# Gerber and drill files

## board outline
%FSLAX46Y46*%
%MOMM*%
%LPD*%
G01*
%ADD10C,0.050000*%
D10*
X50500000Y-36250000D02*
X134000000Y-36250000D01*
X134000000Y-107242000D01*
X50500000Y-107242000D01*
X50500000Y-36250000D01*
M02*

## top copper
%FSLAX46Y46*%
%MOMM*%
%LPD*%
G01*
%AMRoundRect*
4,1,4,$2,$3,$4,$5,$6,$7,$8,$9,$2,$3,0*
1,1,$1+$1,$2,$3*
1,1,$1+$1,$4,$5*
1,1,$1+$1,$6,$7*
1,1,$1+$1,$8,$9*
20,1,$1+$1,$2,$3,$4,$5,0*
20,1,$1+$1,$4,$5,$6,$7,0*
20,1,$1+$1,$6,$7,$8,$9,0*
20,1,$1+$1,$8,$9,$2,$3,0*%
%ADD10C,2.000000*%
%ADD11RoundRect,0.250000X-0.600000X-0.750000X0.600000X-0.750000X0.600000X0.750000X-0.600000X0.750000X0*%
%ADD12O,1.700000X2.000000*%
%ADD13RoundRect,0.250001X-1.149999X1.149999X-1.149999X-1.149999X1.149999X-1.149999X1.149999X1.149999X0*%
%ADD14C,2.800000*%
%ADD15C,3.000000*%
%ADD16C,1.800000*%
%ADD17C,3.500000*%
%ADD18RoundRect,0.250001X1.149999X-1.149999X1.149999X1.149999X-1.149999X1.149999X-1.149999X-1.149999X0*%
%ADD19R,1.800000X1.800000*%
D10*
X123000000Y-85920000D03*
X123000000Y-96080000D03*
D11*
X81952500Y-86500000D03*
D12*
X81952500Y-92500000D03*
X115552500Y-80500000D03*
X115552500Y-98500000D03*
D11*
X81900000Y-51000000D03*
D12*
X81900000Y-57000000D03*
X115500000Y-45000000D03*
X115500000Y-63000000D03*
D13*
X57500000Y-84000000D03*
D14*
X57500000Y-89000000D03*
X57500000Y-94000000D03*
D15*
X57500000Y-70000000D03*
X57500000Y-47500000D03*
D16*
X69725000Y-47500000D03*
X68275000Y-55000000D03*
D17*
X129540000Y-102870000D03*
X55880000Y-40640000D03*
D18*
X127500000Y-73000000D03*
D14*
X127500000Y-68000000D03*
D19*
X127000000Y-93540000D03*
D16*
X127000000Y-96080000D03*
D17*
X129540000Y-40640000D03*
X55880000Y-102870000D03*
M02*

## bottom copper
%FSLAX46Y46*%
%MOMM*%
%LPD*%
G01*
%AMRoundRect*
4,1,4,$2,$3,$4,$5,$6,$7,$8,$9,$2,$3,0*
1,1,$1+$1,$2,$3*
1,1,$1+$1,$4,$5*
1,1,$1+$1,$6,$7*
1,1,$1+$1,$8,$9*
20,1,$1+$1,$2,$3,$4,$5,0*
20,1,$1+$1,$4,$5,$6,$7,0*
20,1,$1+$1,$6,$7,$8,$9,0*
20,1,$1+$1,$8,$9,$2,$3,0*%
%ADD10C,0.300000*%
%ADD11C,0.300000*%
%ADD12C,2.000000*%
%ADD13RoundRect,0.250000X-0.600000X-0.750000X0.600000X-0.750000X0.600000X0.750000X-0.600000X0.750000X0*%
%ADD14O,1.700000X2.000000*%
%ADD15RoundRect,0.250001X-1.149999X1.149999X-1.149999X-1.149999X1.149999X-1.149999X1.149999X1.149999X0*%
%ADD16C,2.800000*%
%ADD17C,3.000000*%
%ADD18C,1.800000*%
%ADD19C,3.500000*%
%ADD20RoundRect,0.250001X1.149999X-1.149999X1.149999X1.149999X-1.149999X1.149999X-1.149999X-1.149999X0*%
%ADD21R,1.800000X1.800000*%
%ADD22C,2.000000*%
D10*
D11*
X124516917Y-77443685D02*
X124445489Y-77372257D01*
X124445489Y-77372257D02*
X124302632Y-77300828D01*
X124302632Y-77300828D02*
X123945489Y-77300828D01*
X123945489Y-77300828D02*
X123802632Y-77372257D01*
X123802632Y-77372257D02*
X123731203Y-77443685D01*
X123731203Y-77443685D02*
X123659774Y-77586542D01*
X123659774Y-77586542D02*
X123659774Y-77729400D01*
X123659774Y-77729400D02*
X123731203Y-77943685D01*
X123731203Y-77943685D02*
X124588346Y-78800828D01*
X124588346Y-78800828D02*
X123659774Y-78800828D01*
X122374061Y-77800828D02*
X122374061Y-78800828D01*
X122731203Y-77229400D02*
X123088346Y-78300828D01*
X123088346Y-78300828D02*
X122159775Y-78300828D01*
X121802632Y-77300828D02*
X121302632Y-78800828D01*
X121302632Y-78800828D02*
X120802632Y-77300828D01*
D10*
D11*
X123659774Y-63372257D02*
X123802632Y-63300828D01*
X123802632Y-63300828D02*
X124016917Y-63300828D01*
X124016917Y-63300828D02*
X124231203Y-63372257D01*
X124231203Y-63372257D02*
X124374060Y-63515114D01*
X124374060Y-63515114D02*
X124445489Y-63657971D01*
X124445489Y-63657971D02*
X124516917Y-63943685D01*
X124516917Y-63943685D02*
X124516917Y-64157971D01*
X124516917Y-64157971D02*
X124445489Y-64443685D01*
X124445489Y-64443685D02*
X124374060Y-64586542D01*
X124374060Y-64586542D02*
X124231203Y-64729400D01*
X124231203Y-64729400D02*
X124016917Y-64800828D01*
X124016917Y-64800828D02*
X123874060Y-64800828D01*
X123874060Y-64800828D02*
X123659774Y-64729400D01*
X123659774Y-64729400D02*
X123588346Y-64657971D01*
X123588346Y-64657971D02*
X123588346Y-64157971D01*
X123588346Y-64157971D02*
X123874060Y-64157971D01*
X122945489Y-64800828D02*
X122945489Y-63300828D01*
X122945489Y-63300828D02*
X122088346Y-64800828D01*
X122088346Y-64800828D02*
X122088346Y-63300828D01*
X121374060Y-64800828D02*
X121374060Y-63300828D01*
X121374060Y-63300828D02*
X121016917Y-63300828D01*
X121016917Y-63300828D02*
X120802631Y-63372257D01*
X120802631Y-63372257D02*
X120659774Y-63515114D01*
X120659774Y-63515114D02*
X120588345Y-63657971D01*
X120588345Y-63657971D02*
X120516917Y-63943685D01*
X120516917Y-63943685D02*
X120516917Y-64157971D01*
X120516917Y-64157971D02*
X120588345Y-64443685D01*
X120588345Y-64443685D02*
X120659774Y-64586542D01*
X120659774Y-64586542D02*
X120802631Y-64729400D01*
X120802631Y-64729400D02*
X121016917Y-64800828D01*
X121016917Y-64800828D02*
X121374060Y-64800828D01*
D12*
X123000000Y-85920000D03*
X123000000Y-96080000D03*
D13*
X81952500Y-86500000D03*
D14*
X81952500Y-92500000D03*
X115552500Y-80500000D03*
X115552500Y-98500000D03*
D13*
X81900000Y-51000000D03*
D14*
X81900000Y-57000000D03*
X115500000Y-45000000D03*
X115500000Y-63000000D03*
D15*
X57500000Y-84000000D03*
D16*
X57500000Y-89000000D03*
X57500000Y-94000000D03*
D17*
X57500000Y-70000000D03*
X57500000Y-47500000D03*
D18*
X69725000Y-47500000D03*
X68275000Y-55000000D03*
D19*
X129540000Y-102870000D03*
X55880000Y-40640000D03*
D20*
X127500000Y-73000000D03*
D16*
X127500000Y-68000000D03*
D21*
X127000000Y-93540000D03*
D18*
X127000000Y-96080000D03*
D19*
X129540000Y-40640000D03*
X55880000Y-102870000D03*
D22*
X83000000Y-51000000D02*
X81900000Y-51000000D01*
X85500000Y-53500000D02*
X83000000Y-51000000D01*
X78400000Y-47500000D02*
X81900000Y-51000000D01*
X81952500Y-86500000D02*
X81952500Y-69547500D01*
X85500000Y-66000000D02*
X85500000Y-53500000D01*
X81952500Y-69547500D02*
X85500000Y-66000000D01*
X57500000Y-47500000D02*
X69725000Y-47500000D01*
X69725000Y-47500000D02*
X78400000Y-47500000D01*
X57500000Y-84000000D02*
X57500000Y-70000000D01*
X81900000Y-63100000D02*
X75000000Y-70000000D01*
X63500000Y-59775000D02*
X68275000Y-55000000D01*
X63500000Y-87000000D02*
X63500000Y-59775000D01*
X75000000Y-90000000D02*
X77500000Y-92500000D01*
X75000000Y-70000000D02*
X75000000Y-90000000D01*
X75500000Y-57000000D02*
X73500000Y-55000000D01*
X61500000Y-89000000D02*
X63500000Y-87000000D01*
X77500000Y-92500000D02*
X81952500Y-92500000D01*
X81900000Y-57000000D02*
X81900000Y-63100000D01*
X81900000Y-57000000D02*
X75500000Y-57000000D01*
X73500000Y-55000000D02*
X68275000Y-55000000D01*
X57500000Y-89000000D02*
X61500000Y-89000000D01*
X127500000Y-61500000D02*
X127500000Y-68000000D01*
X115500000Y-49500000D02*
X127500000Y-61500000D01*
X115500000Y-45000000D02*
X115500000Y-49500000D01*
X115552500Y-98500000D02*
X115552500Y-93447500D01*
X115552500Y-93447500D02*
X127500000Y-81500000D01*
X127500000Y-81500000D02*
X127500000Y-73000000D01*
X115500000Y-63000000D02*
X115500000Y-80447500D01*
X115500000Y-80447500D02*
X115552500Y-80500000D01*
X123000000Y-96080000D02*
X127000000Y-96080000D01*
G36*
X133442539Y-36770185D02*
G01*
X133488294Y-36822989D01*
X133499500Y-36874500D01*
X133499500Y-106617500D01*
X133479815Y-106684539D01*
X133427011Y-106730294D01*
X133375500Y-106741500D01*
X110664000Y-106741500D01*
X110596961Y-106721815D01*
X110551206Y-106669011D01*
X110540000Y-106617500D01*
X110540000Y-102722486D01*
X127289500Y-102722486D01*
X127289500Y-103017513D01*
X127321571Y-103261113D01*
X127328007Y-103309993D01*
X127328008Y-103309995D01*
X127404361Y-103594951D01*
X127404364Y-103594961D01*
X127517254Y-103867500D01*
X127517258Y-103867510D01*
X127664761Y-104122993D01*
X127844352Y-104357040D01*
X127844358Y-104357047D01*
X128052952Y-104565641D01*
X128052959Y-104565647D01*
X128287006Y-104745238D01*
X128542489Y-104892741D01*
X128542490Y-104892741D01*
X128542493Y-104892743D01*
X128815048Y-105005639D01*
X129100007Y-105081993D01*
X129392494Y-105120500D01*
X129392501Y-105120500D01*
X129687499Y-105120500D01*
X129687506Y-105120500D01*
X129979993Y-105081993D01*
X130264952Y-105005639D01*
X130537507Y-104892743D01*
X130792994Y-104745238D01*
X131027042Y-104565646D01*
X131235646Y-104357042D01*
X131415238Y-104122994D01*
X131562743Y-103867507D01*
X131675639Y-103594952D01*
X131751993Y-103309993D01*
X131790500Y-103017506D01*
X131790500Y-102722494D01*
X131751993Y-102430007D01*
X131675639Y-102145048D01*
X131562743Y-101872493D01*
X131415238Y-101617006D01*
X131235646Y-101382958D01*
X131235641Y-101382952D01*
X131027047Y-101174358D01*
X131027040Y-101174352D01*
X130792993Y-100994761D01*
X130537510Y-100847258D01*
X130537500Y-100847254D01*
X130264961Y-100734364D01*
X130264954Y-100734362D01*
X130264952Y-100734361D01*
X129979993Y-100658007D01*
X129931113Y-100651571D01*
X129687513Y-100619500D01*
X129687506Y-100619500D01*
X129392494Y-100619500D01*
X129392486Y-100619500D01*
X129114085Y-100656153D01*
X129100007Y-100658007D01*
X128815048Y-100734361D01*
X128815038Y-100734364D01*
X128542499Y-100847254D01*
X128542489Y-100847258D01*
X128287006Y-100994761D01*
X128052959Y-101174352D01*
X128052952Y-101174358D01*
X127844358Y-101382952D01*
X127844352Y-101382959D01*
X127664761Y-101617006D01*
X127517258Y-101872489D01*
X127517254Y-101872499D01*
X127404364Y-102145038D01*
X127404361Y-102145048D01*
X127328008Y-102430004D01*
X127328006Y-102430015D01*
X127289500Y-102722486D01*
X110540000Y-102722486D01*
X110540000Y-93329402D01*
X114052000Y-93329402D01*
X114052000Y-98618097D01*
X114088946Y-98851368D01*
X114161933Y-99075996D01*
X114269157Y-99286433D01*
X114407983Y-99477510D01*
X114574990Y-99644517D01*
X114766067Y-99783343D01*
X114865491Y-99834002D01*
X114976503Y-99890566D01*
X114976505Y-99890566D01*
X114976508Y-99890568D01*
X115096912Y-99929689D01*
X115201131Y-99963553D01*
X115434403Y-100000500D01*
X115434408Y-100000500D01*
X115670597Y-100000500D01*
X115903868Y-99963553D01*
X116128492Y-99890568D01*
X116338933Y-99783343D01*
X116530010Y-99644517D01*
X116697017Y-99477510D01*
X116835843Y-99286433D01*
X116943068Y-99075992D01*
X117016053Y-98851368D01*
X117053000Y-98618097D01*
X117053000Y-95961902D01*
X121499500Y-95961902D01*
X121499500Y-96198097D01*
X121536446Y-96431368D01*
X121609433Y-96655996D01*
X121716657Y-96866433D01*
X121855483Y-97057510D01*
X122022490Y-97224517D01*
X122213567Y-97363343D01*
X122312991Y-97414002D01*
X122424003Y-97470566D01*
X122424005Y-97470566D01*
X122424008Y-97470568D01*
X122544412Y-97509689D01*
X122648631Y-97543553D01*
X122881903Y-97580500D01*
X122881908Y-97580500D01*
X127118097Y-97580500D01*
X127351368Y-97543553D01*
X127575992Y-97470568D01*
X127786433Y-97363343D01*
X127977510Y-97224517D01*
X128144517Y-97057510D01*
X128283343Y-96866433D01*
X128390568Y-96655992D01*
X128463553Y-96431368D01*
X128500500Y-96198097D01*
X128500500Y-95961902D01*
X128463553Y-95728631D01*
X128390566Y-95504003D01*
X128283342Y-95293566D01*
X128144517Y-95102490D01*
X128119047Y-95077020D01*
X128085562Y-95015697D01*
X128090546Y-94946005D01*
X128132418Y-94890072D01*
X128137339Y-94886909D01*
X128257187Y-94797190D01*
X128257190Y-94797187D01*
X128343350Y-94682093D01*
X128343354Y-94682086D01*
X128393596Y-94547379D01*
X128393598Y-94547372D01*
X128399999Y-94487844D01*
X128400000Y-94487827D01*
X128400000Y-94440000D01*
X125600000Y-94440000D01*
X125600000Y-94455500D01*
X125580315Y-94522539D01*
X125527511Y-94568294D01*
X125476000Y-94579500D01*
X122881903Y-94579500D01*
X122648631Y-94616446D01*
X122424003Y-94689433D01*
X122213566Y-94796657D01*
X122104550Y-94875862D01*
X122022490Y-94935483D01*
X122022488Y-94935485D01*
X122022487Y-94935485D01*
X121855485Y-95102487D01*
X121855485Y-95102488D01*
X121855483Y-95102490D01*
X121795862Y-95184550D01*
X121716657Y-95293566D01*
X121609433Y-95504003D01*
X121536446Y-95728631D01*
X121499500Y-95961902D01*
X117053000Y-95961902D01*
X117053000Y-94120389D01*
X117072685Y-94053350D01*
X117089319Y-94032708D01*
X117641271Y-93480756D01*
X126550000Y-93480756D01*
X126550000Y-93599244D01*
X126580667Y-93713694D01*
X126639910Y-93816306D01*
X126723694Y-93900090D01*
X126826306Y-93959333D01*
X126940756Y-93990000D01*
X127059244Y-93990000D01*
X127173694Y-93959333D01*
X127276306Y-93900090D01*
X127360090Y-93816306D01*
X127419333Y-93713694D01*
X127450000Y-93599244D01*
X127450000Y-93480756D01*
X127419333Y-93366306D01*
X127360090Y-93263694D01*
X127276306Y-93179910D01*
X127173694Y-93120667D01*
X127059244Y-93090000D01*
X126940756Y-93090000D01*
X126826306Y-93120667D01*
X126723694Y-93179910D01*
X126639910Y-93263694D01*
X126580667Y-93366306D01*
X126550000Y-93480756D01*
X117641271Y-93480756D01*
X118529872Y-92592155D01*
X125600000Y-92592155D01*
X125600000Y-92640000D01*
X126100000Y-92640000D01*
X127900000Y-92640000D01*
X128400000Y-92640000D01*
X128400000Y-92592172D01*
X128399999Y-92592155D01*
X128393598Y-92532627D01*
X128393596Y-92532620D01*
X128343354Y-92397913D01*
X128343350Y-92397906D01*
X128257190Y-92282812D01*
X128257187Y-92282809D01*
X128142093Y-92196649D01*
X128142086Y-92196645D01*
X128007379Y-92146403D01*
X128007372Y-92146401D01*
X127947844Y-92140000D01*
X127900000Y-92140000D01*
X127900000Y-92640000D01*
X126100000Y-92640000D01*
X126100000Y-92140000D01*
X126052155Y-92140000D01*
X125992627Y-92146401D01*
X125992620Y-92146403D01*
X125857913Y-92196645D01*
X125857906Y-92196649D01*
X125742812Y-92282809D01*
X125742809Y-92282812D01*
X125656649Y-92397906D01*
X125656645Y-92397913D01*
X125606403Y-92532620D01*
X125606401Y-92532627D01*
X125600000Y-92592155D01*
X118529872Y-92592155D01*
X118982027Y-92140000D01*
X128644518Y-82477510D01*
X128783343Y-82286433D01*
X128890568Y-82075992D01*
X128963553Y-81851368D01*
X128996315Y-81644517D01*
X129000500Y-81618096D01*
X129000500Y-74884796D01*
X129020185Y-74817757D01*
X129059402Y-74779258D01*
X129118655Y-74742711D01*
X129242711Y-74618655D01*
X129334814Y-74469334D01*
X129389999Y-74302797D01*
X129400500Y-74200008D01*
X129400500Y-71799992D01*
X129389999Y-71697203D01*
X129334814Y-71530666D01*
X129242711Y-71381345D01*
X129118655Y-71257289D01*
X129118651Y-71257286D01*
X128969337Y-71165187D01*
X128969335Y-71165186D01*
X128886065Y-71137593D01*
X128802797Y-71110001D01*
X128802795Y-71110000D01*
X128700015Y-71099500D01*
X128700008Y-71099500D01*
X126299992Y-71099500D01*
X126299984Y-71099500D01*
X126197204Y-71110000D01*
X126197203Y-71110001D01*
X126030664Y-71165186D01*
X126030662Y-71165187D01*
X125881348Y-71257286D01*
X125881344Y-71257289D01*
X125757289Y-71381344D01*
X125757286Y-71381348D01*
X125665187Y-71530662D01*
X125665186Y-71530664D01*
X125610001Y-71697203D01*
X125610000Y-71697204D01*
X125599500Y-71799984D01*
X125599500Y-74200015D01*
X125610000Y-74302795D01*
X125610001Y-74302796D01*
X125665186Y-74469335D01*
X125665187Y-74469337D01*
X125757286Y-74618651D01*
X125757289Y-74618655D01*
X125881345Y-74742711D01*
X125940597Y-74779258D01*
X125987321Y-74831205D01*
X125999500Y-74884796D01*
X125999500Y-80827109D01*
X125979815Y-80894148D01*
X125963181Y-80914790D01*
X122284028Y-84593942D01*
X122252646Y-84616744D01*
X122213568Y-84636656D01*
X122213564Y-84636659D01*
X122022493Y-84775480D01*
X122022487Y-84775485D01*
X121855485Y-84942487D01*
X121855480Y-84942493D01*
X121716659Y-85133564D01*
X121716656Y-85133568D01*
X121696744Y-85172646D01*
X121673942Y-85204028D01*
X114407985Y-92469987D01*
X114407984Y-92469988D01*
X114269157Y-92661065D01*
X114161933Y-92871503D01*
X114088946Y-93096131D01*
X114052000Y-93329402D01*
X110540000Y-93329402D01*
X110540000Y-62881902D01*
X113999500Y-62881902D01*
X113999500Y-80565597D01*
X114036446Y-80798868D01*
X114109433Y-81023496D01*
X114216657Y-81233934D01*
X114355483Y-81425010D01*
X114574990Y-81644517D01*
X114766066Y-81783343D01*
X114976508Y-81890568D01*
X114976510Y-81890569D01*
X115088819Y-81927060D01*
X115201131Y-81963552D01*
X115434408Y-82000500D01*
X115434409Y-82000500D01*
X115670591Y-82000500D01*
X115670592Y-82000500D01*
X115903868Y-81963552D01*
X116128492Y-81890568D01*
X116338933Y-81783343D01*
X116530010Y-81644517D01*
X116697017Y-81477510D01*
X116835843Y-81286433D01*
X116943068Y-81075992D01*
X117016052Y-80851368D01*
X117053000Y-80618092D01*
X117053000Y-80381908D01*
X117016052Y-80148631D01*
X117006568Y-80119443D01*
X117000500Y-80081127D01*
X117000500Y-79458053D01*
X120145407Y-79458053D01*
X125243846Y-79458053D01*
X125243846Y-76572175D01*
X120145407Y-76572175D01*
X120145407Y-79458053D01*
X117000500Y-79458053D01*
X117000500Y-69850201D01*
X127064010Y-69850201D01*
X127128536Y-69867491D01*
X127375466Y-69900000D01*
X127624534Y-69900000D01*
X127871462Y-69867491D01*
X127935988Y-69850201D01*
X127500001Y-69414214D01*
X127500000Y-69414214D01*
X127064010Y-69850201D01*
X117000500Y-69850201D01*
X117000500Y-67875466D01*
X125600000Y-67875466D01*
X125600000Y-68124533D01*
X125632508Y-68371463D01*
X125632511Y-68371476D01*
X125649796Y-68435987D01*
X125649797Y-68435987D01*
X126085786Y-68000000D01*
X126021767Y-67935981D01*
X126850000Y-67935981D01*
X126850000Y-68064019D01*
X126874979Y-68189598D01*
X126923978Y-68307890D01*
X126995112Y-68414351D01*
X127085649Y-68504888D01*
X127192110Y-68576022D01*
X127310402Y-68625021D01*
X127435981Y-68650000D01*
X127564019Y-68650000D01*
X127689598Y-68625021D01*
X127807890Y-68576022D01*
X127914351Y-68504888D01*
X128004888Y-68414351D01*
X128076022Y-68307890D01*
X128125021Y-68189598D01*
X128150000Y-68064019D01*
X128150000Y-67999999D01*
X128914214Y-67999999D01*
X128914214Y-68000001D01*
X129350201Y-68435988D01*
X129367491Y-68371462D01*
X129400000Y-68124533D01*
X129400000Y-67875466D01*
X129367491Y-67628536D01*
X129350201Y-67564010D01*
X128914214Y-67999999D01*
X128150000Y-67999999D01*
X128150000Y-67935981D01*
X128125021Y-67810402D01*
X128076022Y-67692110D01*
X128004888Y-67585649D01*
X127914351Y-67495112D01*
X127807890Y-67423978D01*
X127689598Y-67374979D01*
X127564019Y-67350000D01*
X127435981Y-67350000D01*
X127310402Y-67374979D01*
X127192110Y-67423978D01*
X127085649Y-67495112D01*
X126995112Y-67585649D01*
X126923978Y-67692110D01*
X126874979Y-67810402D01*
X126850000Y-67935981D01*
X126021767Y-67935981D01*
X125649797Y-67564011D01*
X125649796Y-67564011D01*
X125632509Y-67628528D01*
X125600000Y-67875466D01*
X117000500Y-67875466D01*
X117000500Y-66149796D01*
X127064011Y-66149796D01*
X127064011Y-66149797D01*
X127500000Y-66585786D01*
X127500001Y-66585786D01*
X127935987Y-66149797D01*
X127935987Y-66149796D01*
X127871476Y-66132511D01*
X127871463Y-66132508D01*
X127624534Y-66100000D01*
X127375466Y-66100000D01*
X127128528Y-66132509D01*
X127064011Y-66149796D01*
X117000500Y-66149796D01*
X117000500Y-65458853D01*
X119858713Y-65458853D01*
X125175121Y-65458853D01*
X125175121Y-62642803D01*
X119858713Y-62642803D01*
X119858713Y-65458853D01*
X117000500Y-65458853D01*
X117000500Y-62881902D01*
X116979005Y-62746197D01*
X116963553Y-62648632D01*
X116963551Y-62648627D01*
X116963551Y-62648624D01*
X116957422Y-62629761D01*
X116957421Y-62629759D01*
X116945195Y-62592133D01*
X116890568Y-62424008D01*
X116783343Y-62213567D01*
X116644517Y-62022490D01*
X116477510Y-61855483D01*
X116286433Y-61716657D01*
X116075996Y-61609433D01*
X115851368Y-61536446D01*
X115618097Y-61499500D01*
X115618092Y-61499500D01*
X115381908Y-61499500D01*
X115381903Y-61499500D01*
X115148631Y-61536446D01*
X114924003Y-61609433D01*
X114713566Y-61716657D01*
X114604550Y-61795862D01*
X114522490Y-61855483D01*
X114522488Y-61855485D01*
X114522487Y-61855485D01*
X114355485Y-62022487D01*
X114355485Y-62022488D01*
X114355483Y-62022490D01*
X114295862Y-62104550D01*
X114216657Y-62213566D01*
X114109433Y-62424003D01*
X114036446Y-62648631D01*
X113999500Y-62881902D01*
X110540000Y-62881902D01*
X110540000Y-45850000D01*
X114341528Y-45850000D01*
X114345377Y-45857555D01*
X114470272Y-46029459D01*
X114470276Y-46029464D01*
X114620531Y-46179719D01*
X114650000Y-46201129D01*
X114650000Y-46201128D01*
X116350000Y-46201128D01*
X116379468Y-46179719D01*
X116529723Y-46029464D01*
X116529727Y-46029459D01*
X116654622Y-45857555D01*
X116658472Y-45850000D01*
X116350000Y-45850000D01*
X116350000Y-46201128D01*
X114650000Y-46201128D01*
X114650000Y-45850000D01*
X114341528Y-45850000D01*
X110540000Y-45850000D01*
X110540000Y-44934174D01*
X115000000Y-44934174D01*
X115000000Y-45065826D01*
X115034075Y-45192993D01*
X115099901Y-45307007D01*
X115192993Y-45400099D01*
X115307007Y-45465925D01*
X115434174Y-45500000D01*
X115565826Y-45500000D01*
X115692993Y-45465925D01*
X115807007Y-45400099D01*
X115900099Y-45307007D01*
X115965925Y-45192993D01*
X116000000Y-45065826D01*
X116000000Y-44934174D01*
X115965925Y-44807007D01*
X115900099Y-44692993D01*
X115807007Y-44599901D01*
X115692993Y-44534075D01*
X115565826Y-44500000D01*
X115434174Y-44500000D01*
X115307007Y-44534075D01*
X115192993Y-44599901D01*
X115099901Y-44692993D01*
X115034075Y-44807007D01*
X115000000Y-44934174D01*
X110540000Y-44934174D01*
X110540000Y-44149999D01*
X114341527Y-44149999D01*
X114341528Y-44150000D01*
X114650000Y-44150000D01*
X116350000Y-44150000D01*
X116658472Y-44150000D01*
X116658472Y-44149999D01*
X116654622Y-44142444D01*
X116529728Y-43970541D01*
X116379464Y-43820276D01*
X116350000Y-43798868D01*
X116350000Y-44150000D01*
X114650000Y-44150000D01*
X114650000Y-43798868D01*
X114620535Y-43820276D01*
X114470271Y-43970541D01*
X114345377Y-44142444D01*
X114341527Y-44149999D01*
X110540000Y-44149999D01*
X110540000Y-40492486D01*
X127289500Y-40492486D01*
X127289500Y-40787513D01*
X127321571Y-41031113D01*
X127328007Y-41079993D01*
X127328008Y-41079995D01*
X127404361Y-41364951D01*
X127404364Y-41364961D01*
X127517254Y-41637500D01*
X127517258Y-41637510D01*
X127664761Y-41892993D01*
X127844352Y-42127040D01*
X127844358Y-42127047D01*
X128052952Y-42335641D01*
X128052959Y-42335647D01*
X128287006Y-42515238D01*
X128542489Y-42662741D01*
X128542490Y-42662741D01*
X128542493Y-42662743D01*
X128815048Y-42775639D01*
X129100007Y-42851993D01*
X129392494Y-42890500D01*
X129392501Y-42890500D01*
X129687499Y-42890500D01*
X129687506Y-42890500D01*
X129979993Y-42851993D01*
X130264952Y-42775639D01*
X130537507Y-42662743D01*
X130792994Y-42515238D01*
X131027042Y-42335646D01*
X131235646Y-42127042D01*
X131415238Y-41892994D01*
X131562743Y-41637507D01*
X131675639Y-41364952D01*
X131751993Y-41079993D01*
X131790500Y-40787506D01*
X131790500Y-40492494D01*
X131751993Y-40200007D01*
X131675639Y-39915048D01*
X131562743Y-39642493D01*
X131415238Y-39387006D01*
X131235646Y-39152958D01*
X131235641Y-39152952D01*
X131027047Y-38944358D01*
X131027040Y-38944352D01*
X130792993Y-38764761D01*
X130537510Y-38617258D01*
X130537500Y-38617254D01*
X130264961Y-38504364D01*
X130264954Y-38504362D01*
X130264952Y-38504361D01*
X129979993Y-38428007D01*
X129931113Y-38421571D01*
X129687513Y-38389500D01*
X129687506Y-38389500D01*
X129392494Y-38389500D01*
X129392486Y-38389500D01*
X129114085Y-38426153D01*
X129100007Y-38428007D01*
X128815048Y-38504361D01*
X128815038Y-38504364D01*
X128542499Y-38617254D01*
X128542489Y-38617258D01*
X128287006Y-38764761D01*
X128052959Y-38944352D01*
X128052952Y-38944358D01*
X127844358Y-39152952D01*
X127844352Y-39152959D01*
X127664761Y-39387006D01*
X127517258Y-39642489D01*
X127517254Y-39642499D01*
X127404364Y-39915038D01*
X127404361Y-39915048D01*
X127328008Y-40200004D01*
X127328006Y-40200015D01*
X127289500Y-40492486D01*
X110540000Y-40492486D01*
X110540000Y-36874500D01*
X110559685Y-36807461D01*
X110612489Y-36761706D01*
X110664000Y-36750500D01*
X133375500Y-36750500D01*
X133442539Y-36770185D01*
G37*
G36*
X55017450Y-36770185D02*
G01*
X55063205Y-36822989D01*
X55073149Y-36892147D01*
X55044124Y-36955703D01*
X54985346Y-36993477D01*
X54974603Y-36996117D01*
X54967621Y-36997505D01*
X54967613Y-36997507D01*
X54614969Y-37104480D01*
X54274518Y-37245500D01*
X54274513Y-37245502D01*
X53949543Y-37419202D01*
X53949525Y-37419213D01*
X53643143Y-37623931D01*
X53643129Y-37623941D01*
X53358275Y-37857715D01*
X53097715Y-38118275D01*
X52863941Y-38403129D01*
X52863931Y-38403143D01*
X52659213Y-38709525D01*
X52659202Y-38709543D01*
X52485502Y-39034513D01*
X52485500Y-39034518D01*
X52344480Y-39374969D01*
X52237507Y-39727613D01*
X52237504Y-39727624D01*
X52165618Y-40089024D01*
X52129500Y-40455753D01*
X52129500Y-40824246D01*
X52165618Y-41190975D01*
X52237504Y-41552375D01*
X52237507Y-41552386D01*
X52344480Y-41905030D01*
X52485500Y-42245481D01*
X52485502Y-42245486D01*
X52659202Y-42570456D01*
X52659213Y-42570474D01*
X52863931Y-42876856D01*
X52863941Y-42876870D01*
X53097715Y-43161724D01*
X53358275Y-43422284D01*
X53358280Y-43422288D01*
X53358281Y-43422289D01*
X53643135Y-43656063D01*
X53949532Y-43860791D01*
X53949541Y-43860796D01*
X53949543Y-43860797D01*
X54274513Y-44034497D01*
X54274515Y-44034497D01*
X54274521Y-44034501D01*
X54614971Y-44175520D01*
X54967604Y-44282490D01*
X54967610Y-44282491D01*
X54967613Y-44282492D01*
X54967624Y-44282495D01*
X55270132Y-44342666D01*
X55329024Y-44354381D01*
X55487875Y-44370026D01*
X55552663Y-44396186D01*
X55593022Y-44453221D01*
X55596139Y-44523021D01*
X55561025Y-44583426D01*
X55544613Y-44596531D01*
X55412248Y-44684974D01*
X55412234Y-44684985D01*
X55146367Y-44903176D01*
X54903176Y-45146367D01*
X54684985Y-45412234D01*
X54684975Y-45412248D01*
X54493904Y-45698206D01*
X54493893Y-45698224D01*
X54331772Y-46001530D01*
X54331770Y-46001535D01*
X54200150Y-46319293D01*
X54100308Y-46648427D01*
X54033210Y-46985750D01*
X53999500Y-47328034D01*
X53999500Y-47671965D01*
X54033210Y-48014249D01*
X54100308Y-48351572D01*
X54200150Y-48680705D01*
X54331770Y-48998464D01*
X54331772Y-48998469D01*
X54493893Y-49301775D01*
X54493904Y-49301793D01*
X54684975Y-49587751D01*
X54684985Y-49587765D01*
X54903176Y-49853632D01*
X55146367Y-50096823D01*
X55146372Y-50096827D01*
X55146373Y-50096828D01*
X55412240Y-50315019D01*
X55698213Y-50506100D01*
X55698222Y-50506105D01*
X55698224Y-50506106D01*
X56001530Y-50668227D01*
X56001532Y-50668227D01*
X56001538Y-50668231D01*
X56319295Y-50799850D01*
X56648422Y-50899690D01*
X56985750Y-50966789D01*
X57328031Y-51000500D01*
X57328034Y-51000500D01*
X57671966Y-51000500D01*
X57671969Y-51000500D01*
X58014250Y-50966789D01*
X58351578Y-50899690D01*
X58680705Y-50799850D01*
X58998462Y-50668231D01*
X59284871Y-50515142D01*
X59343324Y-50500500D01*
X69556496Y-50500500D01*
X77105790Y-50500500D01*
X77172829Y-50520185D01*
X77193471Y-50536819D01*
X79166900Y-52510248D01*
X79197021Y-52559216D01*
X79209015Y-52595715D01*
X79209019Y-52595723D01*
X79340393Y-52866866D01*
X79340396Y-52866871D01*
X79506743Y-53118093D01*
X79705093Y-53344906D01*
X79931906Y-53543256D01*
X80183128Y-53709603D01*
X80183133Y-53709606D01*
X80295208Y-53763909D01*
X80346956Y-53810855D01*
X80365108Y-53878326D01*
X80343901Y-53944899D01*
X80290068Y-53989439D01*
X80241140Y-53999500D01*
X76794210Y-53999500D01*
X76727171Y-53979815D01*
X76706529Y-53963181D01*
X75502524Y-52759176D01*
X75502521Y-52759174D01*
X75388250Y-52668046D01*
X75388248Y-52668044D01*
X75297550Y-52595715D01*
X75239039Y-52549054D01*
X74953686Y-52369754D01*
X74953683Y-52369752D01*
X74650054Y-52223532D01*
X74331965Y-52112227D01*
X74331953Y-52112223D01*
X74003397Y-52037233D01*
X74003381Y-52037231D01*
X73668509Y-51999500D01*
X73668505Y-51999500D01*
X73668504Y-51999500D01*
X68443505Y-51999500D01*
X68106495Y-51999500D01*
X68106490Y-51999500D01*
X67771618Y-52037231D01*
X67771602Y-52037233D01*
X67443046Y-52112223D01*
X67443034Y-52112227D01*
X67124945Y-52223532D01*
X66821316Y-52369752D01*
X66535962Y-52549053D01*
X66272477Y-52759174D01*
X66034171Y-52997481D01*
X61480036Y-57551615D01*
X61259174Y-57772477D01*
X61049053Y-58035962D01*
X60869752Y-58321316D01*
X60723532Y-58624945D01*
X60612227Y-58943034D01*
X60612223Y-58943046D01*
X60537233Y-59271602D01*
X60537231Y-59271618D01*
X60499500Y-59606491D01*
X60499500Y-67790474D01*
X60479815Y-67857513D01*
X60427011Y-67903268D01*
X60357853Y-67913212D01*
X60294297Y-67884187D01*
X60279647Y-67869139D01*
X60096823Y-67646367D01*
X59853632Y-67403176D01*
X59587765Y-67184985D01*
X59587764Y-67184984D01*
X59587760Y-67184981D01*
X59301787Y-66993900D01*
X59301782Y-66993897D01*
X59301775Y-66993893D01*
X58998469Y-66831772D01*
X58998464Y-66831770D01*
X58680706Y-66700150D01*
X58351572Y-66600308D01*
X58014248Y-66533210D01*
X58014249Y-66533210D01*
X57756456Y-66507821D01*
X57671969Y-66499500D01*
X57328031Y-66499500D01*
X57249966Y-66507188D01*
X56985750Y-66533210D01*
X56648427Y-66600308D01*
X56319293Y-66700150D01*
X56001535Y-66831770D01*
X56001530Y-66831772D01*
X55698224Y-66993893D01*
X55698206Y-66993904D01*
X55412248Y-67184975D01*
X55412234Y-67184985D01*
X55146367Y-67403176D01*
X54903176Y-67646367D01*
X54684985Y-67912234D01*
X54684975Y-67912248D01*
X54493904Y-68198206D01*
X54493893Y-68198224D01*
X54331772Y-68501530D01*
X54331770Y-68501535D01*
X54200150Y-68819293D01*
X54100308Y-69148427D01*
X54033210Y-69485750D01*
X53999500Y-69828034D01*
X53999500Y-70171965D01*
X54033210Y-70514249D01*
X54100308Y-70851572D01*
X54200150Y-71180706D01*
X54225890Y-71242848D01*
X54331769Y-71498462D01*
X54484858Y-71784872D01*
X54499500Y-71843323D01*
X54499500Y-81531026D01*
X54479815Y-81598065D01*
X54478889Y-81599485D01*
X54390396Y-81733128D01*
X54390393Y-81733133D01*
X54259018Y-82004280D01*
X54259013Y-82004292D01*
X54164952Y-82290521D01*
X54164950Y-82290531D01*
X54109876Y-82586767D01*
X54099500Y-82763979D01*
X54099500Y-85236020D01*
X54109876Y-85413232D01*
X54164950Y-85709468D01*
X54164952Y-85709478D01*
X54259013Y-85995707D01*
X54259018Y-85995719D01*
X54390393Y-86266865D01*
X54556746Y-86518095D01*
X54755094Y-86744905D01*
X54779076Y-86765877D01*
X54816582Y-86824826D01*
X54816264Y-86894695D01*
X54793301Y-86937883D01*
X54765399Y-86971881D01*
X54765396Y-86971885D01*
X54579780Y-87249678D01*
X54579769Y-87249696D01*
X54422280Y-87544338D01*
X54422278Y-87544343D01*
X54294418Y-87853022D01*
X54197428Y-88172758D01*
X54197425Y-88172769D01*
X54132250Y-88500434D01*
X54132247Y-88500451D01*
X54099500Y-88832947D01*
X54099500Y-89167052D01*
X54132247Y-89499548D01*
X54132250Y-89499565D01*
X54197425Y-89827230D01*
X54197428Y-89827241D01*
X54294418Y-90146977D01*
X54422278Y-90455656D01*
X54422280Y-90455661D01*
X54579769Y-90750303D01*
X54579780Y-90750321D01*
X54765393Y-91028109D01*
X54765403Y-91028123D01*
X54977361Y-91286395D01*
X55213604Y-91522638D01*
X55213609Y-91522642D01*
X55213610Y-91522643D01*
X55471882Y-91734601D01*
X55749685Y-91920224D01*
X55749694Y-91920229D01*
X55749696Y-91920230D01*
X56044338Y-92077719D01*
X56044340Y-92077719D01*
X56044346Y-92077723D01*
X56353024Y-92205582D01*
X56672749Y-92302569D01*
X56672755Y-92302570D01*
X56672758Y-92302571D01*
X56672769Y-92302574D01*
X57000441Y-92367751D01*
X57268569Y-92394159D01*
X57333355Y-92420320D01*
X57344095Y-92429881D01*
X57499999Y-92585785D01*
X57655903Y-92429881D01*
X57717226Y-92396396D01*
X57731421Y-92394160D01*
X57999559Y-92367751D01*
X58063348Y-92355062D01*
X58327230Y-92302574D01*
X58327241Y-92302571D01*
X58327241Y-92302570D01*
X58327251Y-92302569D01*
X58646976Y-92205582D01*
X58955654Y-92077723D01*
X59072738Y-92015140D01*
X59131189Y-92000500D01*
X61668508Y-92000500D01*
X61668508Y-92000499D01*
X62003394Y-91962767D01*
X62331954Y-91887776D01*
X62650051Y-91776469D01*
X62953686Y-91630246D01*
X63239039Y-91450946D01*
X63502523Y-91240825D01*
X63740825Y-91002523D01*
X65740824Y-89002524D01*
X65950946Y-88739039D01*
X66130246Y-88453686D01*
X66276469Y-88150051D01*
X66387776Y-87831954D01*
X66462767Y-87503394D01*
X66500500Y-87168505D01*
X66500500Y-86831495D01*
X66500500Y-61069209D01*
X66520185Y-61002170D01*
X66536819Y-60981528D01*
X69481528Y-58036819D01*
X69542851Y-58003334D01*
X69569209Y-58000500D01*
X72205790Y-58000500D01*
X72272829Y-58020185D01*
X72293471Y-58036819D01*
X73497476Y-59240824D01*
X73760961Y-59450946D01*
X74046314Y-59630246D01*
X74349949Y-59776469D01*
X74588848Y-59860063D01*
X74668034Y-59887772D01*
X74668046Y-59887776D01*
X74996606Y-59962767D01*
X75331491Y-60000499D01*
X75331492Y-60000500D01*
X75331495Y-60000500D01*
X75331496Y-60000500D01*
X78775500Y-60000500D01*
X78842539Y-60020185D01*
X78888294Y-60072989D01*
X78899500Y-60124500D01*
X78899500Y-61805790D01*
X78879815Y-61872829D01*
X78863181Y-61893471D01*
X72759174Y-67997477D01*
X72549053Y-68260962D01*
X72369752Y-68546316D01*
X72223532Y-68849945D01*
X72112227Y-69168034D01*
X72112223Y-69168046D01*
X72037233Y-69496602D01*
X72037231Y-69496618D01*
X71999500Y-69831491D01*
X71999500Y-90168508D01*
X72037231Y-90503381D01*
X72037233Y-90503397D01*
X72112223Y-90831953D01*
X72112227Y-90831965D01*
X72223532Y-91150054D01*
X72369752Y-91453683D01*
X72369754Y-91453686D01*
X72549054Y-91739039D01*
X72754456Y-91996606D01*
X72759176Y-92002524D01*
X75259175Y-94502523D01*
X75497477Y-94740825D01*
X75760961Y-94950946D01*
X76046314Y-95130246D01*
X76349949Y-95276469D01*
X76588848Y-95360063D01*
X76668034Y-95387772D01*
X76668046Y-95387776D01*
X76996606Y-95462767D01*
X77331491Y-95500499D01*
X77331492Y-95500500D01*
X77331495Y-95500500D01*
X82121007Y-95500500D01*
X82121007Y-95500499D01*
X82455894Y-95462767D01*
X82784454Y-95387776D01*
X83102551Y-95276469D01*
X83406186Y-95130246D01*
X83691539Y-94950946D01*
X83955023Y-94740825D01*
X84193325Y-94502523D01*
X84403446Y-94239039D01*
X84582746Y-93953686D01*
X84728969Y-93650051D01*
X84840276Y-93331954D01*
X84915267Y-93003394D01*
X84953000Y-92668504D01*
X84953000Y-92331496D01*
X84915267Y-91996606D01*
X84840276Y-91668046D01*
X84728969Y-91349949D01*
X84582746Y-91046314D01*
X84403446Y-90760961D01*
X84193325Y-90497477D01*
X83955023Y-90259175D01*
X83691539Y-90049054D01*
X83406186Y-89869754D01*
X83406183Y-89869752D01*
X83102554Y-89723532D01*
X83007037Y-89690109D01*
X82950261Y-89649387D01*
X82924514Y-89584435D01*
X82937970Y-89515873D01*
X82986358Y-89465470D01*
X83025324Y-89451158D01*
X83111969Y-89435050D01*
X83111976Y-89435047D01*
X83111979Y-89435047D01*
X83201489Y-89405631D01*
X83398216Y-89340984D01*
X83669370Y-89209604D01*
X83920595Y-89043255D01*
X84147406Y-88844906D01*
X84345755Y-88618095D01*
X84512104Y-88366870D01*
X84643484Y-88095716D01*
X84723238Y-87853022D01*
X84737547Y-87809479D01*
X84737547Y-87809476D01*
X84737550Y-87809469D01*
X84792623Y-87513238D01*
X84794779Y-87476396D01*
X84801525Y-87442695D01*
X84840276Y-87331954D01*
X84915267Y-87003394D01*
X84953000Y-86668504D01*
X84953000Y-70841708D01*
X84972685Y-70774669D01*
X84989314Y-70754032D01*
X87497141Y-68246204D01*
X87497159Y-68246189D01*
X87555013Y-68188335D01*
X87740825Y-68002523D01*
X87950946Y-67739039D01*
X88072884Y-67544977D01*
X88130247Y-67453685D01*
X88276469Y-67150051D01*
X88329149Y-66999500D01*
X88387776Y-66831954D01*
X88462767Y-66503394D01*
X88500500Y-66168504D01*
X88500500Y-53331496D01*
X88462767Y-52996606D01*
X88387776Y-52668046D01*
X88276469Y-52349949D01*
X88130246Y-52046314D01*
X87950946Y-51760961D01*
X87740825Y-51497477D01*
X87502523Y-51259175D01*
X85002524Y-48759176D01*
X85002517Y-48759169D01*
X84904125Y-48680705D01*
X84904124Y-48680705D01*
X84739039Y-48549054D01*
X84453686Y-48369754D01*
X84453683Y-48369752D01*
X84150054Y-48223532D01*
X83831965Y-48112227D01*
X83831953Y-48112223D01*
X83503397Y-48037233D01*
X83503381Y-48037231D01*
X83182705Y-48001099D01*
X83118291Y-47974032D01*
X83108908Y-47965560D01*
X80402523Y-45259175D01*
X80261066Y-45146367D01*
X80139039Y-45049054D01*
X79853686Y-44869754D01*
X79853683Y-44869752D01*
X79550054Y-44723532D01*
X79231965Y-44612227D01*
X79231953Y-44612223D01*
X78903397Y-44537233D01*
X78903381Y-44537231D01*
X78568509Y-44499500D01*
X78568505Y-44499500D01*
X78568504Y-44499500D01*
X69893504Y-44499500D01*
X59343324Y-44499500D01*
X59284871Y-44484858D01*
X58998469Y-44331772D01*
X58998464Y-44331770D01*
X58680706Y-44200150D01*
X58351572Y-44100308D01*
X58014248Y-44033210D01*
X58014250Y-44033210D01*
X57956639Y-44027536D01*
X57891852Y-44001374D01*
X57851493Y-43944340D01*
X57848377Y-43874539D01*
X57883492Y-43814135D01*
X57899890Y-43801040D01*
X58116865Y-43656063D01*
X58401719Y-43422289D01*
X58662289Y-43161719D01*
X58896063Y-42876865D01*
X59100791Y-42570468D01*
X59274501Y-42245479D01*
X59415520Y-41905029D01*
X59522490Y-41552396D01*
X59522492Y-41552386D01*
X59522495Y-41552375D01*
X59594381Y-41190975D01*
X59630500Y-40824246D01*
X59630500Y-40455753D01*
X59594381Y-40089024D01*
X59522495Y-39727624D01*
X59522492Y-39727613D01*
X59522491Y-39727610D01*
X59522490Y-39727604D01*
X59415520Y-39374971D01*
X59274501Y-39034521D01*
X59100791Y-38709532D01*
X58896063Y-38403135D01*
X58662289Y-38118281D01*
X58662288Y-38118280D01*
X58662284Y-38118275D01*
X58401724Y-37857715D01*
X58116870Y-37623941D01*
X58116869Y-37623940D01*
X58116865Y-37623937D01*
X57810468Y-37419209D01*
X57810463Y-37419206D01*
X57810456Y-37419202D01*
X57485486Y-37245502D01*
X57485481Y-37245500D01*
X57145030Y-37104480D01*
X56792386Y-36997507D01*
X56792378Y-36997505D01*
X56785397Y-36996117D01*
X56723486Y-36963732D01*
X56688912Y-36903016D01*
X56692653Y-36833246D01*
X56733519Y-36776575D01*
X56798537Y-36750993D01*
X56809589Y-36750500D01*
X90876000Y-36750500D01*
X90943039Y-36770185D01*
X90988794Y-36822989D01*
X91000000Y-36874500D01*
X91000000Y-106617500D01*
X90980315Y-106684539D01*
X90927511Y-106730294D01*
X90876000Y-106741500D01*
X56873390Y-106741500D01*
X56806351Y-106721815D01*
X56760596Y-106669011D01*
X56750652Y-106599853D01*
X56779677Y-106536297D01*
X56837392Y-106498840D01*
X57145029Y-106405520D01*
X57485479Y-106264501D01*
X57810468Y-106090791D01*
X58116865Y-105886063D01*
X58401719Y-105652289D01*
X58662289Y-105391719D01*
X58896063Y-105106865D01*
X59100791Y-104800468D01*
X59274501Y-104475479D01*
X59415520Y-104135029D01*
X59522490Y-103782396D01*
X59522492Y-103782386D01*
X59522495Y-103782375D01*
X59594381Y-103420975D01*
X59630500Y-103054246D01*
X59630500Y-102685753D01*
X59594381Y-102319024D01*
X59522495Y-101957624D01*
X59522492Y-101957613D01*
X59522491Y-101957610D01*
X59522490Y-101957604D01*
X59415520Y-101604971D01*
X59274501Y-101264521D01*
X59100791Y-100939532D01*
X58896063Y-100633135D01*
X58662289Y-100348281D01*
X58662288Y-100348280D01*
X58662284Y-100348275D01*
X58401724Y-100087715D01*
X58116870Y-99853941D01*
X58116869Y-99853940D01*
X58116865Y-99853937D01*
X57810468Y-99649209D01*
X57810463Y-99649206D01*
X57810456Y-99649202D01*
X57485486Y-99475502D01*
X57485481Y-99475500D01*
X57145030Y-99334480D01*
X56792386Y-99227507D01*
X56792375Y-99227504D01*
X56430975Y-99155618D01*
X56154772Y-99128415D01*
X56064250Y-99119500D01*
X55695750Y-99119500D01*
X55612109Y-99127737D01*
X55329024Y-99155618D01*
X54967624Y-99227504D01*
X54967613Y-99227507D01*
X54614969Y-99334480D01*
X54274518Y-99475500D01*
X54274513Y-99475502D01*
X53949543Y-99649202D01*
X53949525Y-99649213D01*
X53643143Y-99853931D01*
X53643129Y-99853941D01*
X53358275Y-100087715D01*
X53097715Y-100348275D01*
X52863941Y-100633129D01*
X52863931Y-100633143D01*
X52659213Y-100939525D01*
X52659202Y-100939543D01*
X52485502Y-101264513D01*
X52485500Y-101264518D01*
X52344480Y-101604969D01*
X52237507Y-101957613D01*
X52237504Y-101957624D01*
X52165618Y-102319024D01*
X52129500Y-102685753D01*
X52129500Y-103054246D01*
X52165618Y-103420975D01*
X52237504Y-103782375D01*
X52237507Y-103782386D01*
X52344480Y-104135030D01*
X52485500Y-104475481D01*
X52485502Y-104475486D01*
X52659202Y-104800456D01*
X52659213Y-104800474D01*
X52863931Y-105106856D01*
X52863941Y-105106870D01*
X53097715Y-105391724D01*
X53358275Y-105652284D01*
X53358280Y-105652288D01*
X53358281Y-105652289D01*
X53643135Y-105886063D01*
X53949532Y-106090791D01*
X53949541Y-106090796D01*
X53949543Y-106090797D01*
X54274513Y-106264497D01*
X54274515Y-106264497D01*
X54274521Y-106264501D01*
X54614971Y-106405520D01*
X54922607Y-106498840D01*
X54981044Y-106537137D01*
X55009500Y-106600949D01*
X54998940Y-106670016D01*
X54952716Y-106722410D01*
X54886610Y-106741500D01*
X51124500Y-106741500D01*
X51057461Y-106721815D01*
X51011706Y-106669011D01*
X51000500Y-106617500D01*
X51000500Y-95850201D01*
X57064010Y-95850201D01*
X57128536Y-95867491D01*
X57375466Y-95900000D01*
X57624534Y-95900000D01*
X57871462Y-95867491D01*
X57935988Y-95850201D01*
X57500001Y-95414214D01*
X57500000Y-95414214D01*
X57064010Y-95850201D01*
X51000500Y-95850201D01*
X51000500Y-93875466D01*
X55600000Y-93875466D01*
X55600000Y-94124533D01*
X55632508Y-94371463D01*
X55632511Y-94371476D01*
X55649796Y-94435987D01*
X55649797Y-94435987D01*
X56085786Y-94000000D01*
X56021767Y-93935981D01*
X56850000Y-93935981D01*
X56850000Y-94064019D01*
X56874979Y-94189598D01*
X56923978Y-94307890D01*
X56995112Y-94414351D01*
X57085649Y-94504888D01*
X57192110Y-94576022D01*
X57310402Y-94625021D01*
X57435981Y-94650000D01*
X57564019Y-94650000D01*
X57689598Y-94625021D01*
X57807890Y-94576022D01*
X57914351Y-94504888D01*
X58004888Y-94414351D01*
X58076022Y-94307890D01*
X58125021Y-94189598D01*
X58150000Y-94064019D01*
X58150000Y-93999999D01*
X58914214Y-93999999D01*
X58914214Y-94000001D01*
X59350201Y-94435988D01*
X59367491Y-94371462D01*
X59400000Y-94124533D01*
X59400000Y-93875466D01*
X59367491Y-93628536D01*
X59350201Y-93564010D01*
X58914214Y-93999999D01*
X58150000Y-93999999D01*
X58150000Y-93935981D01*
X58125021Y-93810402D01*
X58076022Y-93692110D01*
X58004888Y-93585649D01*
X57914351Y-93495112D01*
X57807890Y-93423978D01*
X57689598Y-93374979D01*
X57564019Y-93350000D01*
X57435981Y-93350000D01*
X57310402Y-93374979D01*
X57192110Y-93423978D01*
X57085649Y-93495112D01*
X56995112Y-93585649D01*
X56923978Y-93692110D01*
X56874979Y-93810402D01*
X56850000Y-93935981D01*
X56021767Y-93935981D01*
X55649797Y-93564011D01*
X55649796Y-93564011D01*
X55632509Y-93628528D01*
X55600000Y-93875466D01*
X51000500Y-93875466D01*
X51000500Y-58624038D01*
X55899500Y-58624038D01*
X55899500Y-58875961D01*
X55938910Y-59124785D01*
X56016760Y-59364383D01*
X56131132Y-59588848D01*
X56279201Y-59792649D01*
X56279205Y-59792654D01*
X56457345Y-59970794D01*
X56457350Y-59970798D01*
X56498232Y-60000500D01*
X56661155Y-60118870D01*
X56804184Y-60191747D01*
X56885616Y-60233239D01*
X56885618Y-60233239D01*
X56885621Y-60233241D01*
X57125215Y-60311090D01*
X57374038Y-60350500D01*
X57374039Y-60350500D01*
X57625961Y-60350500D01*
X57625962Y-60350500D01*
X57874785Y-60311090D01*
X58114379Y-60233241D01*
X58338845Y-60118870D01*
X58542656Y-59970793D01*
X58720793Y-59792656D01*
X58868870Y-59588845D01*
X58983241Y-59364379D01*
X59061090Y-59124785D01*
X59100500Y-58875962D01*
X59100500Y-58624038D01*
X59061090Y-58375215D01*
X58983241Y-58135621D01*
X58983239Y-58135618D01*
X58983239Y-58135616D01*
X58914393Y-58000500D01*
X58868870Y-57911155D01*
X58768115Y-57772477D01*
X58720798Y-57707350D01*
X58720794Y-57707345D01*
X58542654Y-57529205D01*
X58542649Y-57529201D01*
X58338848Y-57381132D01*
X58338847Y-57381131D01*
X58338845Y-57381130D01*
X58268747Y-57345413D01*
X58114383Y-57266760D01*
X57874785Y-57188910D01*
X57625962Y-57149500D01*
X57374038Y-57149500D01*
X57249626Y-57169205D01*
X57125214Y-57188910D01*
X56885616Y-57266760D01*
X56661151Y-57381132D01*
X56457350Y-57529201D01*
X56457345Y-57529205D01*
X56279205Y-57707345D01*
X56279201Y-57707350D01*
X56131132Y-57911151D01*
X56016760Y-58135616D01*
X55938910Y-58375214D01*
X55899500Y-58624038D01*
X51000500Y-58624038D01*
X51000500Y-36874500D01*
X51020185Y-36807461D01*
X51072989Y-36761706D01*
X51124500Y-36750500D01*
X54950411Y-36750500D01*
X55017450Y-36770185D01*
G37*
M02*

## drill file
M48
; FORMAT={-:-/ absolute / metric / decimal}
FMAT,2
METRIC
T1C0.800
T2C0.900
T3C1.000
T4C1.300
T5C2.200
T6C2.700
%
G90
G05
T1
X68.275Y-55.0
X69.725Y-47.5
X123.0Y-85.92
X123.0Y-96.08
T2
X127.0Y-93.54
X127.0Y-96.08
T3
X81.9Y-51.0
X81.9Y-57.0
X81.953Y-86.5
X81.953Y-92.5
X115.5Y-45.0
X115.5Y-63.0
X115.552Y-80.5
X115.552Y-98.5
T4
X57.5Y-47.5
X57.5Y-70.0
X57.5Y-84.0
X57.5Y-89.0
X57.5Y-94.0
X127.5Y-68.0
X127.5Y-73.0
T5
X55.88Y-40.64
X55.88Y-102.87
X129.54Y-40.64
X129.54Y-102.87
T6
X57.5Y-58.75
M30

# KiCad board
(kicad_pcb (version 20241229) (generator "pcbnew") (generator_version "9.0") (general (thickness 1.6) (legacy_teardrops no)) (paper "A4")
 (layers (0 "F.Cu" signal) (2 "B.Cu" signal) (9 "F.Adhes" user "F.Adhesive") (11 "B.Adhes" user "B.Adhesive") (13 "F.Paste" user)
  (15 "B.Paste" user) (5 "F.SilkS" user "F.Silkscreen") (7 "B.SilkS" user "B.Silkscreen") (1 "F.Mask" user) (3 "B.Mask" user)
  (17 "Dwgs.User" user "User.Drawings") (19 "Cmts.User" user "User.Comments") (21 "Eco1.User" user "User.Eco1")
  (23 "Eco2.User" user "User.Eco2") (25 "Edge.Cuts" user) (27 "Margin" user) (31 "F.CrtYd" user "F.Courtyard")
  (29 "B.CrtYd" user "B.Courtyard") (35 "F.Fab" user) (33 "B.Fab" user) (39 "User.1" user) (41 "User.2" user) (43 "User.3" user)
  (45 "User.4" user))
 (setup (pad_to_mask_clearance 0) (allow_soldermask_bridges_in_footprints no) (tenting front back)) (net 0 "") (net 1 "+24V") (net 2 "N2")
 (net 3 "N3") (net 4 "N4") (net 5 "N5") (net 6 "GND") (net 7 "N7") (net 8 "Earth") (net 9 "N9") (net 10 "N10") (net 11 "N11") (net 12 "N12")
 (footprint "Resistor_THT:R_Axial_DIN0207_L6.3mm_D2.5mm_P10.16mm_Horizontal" (layer "F.Cu") (at 123 85.92 -90)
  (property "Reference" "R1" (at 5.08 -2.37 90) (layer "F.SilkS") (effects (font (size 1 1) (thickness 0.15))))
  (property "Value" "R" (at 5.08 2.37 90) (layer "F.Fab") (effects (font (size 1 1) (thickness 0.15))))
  (pad "1" thru_hole circle (at 0 0 270) (size 2 2) (drill 0.8) (layers "*.Cu" "*.Mask") (remove_unused_layers no) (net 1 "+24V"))
  (pad "2" thru_hole circle (at 10.16 0 270) (size 2 2) (drill 0.8) (layers "*.Cu" "*.Mask") (remove_unused_layers no) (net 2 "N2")))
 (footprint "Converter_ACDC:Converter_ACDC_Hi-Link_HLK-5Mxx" (layer "F.Cu") (at 81.9525 86.5)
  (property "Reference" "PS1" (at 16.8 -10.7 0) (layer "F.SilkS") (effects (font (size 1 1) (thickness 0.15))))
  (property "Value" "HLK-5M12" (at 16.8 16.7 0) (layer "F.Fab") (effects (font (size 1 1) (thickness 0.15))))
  (pad "1" thru_hole roundrect (at 0 0) (size 1.7 2) (drill 1) (layers "*.Cu" "*.Mask") (remove_unused_layers no)
   (roundrect_rratio 0.147059) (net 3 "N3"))
  (pad "2" thru_hole oval (at 0 6) (size 1.7 2) (drill 1) (layers "*.Cu" "*.Mask") (remove_unused_layers no) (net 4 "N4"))
  (pad "3" thru_hole oval (at 33.6 -6) (size 1.7 2) (drill 1) (layers "*.Cu" "*.Mask") (remove_unused_layers no) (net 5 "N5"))
  (pad "4" thru_hole oval (at 33.6 12) (size 1.7 2) (drill 1) (layers "*.Cu" "*.Mask") (remove_unused_layers no) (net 1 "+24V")))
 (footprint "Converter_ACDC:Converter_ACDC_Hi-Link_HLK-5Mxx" (layer "F.Cu") (at 81.9 51)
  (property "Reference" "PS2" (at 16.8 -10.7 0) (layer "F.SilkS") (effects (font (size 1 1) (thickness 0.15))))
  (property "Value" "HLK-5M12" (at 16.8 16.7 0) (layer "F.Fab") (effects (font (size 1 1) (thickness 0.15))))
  (pad "1" thru_hole roundrect (at 0 0) (size 1.7 2) (drill 1) (layers "*.Cu" "*.Mask") (remove_unused_layers no)
   (roundrect_rratio 0.147059) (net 3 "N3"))
  (pad "2" thru_hole oval (at 0 6) (size 1.7 2) (drill 1) (layers "*.Cu" "*.Mask") (remove_unused_layers no) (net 4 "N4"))
  (pad "3" thru_hole oval (at 33.6 -6) (size 1.7 2) (drill 1) (layers "*.Cu" "*.Mask") (remove_unused_layers no) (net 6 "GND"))
  (pad "4" thru_hole oval (at 33.6 12) (size 1.7 2) (drill 1) (layers "*.Cu" "*.Mask") (remove_unused_layers no) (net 5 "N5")))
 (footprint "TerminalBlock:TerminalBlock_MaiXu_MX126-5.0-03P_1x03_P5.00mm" (layer "F.Cu") (at 57.5 84 -90)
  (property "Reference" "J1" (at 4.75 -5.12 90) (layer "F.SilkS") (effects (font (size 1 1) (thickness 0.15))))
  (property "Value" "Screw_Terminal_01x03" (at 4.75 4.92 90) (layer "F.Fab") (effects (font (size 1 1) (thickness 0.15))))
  (pad "1" thru_hole roundrect (at 0 0 270) (size 2.8 2.8) (drill 1.3) (layers "*.Cu" "*.Mask") (remove_unused_layers no)
   (roundrect_rratio 0.089286) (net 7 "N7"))
  (pad "2" thru_hole circle (at 5 0 270) (size 2.8 2.8) (drill 1.3) (layers "*.Cu" "*.Mask") (remove_unused_layers no) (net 4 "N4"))
  (pad "3" thru_hole circle (at 10 0 270) (size 2.8 2.8) (drill 1.3) (layers "*.Cu" "*.Mask") (remove_unused_layers no) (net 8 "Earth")))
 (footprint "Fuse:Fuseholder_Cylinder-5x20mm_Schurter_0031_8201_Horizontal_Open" (layer "F.Cu") (at 57.5 70 90)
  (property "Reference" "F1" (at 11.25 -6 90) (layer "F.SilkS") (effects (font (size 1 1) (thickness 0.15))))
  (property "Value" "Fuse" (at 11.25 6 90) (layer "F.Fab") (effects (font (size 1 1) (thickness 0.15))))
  (pad "" np_thru_hole circle (at 11.25 0 90) (size 2.7 2.7) (drill 2.7) (layers "*.Cu" "*.Mask"))
  (pad "1" thru_hole circle (at 0 0 90) (size 3 3) (drill 1.3) (layers "*.Cu" "*.Mask") (remove_unused_layers no) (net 7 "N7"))
  (pad "2" thru_hole circle (at 22.5 0 90) (size 3 3) (drill 1.3) (layers "*.Cu" "*.Mask") (remove_unused_layers no) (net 3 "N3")))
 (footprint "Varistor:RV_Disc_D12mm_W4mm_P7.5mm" (layer "F.Cu") (at 69.725 47.5 -90)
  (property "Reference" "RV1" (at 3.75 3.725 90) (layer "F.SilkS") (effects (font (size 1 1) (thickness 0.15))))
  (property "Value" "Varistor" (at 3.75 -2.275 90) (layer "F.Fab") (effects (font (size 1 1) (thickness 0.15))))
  (pad "1" thru_hole circle (at 0 0 270) (size 1.8 1.8) (drill 0.8) (layers "*.Cu" "*.Mask") (remove_unused_layers no) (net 3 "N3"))
  (pad "2" thru_hole circle (at 7.5 1.45 270) (size 1.8 1.8) (drill 0.8) (layers "*.Cu" "*.Mask") (remove_unused_layers no) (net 4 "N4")))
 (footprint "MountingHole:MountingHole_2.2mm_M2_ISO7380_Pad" (layer "F.Cu") (at 129.54 102.87)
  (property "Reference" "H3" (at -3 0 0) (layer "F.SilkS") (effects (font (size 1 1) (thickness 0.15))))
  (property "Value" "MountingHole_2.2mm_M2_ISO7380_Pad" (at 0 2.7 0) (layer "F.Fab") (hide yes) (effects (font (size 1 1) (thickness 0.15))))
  (pad "1" thru_hole circle (at 0 0) (size 3.5 3.5) (drill 2.2) (layers "*.Cu" "*.Mask") (remove_unused_layers no) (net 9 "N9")
   (zone_connect 2)))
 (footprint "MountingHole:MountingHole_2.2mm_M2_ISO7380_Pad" (layer "F.Cu") (at 55.88 40.64)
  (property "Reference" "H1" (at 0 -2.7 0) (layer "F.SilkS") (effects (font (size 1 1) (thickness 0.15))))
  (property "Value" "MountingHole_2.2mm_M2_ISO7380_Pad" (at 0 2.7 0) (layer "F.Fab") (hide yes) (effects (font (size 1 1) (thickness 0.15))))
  (pad "1" thru_hole circle (at 0 0) (size 3.5 3.5) (drill 2.2) (layers "*.Cu" "*.Mask") (remove_unused_layers no) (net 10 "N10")
   (zone_connect 2)))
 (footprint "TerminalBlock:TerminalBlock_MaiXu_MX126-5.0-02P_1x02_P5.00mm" (layer "F.Cu") (at 127.5 73 90)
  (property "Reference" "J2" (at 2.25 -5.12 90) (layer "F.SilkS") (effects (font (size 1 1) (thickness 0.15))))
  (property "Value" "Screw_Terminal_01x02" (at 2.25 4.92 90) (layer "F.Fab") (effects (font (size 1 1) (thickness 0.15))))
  (pad "1" thru_hole roundrect (at 0 0 90) (size 2.8 2.8) (drill 1.3) (layers "*.Cu" "*.Mask") (remove_unused_layers no)
   (roundrect_rratio 0.089286) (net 1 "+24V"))
  (pad "2" thru_hole circle (at 5 0 90) (size 2.8 2.8) (drill 1.3) (layers "*.Cu" "*.Mask") (remove_unused_layers no) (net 6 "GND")))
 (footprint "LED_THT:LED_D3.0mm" (layer "F.Cu") (at 127 93.54 -90)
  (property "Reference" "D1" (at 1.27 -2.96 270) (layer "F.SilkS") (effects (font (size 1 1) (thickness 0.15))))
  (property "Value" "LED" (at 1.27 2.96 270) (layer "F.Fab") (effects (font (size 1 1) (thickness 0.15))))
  (pad "1" thru_hole rect (at 0 0 270) (size 1.8 1.8) (drill 0.9) (layers "*.Cu" "*.Mask") (remove_unused_layers no) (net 6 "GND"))
  (pad "2" thru_hole circle (at 2.54 0 270) (size 1.8 1.8) (drill 0.9) (layers "*.Cu" "*.Mask") (remove_unused_layers no) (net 2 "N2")))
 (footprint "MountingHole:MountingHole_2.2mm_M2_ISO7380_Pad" (layer "F.Cu") (at 129.54 40.64)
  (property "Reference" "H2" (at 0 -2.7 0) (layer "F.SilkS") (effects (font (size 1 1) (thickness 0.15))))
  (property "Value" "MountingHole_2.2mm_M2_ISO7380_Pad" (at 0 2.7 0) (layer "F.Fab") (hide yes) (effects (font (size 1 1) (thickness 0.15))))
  (pad "1" thru_hole circle (at 0 0) (size 3.5 3.5) (drill 2.2) (layers "*.Cu" "*.Mask") (remove_unused_layers no) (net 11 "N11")
   (zone_connect 2)))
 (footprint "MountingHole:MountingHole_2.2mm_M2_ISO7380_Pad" (layer "F.Cu") (at 55.88 102.87)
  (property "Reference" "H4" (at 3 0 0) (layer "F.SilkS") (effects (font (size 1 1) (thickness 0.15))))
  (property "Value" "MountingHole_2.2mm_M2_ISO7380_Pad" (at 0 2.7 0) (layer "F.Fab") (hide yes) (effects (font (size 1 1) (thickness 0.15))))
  (pad "1" thru_hole circle (at 0 0) (size 3.5 3.5) (drill 2.2) (layers "*.Cu" "*.Mask") (remove_unused_layers no) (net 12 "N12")
   (zone_connect 2)))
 (gr_rect (start 50.5 36.25) (end 134 107.242) (stroke (width 0.05) (type default)) (fill no) (layer "Edge.Cuts"))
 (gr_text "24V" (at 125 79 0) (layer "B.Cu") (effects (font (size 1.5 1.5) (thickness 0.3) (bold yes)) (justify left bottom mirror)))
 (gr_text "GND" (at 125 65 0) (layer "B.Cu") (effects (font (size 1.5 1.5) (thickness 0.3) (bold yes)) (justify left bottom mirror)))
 (segment (start 83 51) (end 81.9 51) (width 2) (layer "B.Cu") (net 3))
 (segment (start 85.5 53.5) (end 83 51) (width 2) (layer "B.Cu") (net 3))
 (segment (start 78.4 47.5) (end 81.9 51) (width 2) (layer "B.Cu") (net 3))
 (segment (start 81.9525 86.5) (end 81.9525 69.5475) (width 2) (layer "B.Cu") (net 3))
 (segment (start 85.5 66) (end 85.5 53.5) (width 2) (layer "B.Cu") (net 3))
 (segment (start 81.9525 69.5475) (end 85.5 66) (width 2) (layer "B.Cu") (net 3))
 (segment (start 57.5 47.5) (end 69.725 47.5) (width 2) (layer "B.Cu") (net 3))
 (segment (start 69.725 47.5) (end 78.4 47.5) (width 2) (layer "B.Cu") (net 3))
 (segment (start 57.5 84) (end 57.5 70) (width 2) (layer "B.Cu") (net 7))
 (segment (start 81.9 63.1) (end 75 70) (width 2) (layer "B.Cu") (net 4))
 (segment (start 63.5 59.775) (end 68.275 55) (width 2) (layer "B.Cu") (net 4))
 (segment (start 63.5 87) (end 63.5 59.775) (width 2) (layer "B.Cu") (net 4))
 (segment (start 75 90) (end 77.5 92.5) (width 2) (layer "B.Cu") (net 4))
 (segment (start 75 70) (end 75 90) (width 2) (layer "B.Cu") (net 4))
 (segment (start 75.5 57) (end 73.5 55) (width 2) (layer "B.Cu") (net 4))
 (segment (start 61.5 89) (end 63.5 87) (width 2) (layer "B.Cu") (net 4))
 (segment (start 77.5 92.5) (end 81.9525 92.5) (width 2) (layer "B.Cu") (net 4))
 (segment (start 81.9 57) (end 81.9 63.1) (width 2) (layer "B.Cu") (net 4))
 (segment (start 81.9 57) (end 75.5 57) (width 2) (layer "B.Cu") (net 4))
 (segment (start 73.5 55) (end 68.275 55) (width 2) (layer "B.Cu") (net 4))
 (segment (start 57.5 89) (end 61.5 89) (width 2) (layer "B.Cu") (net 4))
 (segment (start 127.5 61.5) (end 127.5 68) (width 2) (layer "B.Cu") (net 6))
 (segment (start 115.5 49.5) (end 127.5 61.5) (width 2) (layer "B.Cu") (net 6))
 (segment (start 115.5 45) (end 115.5 49.5) (width 2) (layer "B.Cu") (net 6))
 (segment (start 115.5525 98.5) (end 115.5525 93.4475) (width 2) (layer "B.Cu") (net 1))
 (segment (start 115.5525 93.4475) (end 127.5 81.5) (width 2) (layer "B.Cu") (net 1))
 (segment (start 127.5 81.5) (end 127.5 73) (width 2) (layer "B.Cu") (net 1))
 (segment (start 115.5 63) (end 115.5 80.4475) (width 2) (layer "B.Cu") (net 5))
 (segment (start 115.5 80.4475) (end 115.5525 80.5) (width 2) (layer "B.Cu") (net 5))
 (segment (start 123 96.08) (end 127 96.08) (width 2) (layer "B.Cu") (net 2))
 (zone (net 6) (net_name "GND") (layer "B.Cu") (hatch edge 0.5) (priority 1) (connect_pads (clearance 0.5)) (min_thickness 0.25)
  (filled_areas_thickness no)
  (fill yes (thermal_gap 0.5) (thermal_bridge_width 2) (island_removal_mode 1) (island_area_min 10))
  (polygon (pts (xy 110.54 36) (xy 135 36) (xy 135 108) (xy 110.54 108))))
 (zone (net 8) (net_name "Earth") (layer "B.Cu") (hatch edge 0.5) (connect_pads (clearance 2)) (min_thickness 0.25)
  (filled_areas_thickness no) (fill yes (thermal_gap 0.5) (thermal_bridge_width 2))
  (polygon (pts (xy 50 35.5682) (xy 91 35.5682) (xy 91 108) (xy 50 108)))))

